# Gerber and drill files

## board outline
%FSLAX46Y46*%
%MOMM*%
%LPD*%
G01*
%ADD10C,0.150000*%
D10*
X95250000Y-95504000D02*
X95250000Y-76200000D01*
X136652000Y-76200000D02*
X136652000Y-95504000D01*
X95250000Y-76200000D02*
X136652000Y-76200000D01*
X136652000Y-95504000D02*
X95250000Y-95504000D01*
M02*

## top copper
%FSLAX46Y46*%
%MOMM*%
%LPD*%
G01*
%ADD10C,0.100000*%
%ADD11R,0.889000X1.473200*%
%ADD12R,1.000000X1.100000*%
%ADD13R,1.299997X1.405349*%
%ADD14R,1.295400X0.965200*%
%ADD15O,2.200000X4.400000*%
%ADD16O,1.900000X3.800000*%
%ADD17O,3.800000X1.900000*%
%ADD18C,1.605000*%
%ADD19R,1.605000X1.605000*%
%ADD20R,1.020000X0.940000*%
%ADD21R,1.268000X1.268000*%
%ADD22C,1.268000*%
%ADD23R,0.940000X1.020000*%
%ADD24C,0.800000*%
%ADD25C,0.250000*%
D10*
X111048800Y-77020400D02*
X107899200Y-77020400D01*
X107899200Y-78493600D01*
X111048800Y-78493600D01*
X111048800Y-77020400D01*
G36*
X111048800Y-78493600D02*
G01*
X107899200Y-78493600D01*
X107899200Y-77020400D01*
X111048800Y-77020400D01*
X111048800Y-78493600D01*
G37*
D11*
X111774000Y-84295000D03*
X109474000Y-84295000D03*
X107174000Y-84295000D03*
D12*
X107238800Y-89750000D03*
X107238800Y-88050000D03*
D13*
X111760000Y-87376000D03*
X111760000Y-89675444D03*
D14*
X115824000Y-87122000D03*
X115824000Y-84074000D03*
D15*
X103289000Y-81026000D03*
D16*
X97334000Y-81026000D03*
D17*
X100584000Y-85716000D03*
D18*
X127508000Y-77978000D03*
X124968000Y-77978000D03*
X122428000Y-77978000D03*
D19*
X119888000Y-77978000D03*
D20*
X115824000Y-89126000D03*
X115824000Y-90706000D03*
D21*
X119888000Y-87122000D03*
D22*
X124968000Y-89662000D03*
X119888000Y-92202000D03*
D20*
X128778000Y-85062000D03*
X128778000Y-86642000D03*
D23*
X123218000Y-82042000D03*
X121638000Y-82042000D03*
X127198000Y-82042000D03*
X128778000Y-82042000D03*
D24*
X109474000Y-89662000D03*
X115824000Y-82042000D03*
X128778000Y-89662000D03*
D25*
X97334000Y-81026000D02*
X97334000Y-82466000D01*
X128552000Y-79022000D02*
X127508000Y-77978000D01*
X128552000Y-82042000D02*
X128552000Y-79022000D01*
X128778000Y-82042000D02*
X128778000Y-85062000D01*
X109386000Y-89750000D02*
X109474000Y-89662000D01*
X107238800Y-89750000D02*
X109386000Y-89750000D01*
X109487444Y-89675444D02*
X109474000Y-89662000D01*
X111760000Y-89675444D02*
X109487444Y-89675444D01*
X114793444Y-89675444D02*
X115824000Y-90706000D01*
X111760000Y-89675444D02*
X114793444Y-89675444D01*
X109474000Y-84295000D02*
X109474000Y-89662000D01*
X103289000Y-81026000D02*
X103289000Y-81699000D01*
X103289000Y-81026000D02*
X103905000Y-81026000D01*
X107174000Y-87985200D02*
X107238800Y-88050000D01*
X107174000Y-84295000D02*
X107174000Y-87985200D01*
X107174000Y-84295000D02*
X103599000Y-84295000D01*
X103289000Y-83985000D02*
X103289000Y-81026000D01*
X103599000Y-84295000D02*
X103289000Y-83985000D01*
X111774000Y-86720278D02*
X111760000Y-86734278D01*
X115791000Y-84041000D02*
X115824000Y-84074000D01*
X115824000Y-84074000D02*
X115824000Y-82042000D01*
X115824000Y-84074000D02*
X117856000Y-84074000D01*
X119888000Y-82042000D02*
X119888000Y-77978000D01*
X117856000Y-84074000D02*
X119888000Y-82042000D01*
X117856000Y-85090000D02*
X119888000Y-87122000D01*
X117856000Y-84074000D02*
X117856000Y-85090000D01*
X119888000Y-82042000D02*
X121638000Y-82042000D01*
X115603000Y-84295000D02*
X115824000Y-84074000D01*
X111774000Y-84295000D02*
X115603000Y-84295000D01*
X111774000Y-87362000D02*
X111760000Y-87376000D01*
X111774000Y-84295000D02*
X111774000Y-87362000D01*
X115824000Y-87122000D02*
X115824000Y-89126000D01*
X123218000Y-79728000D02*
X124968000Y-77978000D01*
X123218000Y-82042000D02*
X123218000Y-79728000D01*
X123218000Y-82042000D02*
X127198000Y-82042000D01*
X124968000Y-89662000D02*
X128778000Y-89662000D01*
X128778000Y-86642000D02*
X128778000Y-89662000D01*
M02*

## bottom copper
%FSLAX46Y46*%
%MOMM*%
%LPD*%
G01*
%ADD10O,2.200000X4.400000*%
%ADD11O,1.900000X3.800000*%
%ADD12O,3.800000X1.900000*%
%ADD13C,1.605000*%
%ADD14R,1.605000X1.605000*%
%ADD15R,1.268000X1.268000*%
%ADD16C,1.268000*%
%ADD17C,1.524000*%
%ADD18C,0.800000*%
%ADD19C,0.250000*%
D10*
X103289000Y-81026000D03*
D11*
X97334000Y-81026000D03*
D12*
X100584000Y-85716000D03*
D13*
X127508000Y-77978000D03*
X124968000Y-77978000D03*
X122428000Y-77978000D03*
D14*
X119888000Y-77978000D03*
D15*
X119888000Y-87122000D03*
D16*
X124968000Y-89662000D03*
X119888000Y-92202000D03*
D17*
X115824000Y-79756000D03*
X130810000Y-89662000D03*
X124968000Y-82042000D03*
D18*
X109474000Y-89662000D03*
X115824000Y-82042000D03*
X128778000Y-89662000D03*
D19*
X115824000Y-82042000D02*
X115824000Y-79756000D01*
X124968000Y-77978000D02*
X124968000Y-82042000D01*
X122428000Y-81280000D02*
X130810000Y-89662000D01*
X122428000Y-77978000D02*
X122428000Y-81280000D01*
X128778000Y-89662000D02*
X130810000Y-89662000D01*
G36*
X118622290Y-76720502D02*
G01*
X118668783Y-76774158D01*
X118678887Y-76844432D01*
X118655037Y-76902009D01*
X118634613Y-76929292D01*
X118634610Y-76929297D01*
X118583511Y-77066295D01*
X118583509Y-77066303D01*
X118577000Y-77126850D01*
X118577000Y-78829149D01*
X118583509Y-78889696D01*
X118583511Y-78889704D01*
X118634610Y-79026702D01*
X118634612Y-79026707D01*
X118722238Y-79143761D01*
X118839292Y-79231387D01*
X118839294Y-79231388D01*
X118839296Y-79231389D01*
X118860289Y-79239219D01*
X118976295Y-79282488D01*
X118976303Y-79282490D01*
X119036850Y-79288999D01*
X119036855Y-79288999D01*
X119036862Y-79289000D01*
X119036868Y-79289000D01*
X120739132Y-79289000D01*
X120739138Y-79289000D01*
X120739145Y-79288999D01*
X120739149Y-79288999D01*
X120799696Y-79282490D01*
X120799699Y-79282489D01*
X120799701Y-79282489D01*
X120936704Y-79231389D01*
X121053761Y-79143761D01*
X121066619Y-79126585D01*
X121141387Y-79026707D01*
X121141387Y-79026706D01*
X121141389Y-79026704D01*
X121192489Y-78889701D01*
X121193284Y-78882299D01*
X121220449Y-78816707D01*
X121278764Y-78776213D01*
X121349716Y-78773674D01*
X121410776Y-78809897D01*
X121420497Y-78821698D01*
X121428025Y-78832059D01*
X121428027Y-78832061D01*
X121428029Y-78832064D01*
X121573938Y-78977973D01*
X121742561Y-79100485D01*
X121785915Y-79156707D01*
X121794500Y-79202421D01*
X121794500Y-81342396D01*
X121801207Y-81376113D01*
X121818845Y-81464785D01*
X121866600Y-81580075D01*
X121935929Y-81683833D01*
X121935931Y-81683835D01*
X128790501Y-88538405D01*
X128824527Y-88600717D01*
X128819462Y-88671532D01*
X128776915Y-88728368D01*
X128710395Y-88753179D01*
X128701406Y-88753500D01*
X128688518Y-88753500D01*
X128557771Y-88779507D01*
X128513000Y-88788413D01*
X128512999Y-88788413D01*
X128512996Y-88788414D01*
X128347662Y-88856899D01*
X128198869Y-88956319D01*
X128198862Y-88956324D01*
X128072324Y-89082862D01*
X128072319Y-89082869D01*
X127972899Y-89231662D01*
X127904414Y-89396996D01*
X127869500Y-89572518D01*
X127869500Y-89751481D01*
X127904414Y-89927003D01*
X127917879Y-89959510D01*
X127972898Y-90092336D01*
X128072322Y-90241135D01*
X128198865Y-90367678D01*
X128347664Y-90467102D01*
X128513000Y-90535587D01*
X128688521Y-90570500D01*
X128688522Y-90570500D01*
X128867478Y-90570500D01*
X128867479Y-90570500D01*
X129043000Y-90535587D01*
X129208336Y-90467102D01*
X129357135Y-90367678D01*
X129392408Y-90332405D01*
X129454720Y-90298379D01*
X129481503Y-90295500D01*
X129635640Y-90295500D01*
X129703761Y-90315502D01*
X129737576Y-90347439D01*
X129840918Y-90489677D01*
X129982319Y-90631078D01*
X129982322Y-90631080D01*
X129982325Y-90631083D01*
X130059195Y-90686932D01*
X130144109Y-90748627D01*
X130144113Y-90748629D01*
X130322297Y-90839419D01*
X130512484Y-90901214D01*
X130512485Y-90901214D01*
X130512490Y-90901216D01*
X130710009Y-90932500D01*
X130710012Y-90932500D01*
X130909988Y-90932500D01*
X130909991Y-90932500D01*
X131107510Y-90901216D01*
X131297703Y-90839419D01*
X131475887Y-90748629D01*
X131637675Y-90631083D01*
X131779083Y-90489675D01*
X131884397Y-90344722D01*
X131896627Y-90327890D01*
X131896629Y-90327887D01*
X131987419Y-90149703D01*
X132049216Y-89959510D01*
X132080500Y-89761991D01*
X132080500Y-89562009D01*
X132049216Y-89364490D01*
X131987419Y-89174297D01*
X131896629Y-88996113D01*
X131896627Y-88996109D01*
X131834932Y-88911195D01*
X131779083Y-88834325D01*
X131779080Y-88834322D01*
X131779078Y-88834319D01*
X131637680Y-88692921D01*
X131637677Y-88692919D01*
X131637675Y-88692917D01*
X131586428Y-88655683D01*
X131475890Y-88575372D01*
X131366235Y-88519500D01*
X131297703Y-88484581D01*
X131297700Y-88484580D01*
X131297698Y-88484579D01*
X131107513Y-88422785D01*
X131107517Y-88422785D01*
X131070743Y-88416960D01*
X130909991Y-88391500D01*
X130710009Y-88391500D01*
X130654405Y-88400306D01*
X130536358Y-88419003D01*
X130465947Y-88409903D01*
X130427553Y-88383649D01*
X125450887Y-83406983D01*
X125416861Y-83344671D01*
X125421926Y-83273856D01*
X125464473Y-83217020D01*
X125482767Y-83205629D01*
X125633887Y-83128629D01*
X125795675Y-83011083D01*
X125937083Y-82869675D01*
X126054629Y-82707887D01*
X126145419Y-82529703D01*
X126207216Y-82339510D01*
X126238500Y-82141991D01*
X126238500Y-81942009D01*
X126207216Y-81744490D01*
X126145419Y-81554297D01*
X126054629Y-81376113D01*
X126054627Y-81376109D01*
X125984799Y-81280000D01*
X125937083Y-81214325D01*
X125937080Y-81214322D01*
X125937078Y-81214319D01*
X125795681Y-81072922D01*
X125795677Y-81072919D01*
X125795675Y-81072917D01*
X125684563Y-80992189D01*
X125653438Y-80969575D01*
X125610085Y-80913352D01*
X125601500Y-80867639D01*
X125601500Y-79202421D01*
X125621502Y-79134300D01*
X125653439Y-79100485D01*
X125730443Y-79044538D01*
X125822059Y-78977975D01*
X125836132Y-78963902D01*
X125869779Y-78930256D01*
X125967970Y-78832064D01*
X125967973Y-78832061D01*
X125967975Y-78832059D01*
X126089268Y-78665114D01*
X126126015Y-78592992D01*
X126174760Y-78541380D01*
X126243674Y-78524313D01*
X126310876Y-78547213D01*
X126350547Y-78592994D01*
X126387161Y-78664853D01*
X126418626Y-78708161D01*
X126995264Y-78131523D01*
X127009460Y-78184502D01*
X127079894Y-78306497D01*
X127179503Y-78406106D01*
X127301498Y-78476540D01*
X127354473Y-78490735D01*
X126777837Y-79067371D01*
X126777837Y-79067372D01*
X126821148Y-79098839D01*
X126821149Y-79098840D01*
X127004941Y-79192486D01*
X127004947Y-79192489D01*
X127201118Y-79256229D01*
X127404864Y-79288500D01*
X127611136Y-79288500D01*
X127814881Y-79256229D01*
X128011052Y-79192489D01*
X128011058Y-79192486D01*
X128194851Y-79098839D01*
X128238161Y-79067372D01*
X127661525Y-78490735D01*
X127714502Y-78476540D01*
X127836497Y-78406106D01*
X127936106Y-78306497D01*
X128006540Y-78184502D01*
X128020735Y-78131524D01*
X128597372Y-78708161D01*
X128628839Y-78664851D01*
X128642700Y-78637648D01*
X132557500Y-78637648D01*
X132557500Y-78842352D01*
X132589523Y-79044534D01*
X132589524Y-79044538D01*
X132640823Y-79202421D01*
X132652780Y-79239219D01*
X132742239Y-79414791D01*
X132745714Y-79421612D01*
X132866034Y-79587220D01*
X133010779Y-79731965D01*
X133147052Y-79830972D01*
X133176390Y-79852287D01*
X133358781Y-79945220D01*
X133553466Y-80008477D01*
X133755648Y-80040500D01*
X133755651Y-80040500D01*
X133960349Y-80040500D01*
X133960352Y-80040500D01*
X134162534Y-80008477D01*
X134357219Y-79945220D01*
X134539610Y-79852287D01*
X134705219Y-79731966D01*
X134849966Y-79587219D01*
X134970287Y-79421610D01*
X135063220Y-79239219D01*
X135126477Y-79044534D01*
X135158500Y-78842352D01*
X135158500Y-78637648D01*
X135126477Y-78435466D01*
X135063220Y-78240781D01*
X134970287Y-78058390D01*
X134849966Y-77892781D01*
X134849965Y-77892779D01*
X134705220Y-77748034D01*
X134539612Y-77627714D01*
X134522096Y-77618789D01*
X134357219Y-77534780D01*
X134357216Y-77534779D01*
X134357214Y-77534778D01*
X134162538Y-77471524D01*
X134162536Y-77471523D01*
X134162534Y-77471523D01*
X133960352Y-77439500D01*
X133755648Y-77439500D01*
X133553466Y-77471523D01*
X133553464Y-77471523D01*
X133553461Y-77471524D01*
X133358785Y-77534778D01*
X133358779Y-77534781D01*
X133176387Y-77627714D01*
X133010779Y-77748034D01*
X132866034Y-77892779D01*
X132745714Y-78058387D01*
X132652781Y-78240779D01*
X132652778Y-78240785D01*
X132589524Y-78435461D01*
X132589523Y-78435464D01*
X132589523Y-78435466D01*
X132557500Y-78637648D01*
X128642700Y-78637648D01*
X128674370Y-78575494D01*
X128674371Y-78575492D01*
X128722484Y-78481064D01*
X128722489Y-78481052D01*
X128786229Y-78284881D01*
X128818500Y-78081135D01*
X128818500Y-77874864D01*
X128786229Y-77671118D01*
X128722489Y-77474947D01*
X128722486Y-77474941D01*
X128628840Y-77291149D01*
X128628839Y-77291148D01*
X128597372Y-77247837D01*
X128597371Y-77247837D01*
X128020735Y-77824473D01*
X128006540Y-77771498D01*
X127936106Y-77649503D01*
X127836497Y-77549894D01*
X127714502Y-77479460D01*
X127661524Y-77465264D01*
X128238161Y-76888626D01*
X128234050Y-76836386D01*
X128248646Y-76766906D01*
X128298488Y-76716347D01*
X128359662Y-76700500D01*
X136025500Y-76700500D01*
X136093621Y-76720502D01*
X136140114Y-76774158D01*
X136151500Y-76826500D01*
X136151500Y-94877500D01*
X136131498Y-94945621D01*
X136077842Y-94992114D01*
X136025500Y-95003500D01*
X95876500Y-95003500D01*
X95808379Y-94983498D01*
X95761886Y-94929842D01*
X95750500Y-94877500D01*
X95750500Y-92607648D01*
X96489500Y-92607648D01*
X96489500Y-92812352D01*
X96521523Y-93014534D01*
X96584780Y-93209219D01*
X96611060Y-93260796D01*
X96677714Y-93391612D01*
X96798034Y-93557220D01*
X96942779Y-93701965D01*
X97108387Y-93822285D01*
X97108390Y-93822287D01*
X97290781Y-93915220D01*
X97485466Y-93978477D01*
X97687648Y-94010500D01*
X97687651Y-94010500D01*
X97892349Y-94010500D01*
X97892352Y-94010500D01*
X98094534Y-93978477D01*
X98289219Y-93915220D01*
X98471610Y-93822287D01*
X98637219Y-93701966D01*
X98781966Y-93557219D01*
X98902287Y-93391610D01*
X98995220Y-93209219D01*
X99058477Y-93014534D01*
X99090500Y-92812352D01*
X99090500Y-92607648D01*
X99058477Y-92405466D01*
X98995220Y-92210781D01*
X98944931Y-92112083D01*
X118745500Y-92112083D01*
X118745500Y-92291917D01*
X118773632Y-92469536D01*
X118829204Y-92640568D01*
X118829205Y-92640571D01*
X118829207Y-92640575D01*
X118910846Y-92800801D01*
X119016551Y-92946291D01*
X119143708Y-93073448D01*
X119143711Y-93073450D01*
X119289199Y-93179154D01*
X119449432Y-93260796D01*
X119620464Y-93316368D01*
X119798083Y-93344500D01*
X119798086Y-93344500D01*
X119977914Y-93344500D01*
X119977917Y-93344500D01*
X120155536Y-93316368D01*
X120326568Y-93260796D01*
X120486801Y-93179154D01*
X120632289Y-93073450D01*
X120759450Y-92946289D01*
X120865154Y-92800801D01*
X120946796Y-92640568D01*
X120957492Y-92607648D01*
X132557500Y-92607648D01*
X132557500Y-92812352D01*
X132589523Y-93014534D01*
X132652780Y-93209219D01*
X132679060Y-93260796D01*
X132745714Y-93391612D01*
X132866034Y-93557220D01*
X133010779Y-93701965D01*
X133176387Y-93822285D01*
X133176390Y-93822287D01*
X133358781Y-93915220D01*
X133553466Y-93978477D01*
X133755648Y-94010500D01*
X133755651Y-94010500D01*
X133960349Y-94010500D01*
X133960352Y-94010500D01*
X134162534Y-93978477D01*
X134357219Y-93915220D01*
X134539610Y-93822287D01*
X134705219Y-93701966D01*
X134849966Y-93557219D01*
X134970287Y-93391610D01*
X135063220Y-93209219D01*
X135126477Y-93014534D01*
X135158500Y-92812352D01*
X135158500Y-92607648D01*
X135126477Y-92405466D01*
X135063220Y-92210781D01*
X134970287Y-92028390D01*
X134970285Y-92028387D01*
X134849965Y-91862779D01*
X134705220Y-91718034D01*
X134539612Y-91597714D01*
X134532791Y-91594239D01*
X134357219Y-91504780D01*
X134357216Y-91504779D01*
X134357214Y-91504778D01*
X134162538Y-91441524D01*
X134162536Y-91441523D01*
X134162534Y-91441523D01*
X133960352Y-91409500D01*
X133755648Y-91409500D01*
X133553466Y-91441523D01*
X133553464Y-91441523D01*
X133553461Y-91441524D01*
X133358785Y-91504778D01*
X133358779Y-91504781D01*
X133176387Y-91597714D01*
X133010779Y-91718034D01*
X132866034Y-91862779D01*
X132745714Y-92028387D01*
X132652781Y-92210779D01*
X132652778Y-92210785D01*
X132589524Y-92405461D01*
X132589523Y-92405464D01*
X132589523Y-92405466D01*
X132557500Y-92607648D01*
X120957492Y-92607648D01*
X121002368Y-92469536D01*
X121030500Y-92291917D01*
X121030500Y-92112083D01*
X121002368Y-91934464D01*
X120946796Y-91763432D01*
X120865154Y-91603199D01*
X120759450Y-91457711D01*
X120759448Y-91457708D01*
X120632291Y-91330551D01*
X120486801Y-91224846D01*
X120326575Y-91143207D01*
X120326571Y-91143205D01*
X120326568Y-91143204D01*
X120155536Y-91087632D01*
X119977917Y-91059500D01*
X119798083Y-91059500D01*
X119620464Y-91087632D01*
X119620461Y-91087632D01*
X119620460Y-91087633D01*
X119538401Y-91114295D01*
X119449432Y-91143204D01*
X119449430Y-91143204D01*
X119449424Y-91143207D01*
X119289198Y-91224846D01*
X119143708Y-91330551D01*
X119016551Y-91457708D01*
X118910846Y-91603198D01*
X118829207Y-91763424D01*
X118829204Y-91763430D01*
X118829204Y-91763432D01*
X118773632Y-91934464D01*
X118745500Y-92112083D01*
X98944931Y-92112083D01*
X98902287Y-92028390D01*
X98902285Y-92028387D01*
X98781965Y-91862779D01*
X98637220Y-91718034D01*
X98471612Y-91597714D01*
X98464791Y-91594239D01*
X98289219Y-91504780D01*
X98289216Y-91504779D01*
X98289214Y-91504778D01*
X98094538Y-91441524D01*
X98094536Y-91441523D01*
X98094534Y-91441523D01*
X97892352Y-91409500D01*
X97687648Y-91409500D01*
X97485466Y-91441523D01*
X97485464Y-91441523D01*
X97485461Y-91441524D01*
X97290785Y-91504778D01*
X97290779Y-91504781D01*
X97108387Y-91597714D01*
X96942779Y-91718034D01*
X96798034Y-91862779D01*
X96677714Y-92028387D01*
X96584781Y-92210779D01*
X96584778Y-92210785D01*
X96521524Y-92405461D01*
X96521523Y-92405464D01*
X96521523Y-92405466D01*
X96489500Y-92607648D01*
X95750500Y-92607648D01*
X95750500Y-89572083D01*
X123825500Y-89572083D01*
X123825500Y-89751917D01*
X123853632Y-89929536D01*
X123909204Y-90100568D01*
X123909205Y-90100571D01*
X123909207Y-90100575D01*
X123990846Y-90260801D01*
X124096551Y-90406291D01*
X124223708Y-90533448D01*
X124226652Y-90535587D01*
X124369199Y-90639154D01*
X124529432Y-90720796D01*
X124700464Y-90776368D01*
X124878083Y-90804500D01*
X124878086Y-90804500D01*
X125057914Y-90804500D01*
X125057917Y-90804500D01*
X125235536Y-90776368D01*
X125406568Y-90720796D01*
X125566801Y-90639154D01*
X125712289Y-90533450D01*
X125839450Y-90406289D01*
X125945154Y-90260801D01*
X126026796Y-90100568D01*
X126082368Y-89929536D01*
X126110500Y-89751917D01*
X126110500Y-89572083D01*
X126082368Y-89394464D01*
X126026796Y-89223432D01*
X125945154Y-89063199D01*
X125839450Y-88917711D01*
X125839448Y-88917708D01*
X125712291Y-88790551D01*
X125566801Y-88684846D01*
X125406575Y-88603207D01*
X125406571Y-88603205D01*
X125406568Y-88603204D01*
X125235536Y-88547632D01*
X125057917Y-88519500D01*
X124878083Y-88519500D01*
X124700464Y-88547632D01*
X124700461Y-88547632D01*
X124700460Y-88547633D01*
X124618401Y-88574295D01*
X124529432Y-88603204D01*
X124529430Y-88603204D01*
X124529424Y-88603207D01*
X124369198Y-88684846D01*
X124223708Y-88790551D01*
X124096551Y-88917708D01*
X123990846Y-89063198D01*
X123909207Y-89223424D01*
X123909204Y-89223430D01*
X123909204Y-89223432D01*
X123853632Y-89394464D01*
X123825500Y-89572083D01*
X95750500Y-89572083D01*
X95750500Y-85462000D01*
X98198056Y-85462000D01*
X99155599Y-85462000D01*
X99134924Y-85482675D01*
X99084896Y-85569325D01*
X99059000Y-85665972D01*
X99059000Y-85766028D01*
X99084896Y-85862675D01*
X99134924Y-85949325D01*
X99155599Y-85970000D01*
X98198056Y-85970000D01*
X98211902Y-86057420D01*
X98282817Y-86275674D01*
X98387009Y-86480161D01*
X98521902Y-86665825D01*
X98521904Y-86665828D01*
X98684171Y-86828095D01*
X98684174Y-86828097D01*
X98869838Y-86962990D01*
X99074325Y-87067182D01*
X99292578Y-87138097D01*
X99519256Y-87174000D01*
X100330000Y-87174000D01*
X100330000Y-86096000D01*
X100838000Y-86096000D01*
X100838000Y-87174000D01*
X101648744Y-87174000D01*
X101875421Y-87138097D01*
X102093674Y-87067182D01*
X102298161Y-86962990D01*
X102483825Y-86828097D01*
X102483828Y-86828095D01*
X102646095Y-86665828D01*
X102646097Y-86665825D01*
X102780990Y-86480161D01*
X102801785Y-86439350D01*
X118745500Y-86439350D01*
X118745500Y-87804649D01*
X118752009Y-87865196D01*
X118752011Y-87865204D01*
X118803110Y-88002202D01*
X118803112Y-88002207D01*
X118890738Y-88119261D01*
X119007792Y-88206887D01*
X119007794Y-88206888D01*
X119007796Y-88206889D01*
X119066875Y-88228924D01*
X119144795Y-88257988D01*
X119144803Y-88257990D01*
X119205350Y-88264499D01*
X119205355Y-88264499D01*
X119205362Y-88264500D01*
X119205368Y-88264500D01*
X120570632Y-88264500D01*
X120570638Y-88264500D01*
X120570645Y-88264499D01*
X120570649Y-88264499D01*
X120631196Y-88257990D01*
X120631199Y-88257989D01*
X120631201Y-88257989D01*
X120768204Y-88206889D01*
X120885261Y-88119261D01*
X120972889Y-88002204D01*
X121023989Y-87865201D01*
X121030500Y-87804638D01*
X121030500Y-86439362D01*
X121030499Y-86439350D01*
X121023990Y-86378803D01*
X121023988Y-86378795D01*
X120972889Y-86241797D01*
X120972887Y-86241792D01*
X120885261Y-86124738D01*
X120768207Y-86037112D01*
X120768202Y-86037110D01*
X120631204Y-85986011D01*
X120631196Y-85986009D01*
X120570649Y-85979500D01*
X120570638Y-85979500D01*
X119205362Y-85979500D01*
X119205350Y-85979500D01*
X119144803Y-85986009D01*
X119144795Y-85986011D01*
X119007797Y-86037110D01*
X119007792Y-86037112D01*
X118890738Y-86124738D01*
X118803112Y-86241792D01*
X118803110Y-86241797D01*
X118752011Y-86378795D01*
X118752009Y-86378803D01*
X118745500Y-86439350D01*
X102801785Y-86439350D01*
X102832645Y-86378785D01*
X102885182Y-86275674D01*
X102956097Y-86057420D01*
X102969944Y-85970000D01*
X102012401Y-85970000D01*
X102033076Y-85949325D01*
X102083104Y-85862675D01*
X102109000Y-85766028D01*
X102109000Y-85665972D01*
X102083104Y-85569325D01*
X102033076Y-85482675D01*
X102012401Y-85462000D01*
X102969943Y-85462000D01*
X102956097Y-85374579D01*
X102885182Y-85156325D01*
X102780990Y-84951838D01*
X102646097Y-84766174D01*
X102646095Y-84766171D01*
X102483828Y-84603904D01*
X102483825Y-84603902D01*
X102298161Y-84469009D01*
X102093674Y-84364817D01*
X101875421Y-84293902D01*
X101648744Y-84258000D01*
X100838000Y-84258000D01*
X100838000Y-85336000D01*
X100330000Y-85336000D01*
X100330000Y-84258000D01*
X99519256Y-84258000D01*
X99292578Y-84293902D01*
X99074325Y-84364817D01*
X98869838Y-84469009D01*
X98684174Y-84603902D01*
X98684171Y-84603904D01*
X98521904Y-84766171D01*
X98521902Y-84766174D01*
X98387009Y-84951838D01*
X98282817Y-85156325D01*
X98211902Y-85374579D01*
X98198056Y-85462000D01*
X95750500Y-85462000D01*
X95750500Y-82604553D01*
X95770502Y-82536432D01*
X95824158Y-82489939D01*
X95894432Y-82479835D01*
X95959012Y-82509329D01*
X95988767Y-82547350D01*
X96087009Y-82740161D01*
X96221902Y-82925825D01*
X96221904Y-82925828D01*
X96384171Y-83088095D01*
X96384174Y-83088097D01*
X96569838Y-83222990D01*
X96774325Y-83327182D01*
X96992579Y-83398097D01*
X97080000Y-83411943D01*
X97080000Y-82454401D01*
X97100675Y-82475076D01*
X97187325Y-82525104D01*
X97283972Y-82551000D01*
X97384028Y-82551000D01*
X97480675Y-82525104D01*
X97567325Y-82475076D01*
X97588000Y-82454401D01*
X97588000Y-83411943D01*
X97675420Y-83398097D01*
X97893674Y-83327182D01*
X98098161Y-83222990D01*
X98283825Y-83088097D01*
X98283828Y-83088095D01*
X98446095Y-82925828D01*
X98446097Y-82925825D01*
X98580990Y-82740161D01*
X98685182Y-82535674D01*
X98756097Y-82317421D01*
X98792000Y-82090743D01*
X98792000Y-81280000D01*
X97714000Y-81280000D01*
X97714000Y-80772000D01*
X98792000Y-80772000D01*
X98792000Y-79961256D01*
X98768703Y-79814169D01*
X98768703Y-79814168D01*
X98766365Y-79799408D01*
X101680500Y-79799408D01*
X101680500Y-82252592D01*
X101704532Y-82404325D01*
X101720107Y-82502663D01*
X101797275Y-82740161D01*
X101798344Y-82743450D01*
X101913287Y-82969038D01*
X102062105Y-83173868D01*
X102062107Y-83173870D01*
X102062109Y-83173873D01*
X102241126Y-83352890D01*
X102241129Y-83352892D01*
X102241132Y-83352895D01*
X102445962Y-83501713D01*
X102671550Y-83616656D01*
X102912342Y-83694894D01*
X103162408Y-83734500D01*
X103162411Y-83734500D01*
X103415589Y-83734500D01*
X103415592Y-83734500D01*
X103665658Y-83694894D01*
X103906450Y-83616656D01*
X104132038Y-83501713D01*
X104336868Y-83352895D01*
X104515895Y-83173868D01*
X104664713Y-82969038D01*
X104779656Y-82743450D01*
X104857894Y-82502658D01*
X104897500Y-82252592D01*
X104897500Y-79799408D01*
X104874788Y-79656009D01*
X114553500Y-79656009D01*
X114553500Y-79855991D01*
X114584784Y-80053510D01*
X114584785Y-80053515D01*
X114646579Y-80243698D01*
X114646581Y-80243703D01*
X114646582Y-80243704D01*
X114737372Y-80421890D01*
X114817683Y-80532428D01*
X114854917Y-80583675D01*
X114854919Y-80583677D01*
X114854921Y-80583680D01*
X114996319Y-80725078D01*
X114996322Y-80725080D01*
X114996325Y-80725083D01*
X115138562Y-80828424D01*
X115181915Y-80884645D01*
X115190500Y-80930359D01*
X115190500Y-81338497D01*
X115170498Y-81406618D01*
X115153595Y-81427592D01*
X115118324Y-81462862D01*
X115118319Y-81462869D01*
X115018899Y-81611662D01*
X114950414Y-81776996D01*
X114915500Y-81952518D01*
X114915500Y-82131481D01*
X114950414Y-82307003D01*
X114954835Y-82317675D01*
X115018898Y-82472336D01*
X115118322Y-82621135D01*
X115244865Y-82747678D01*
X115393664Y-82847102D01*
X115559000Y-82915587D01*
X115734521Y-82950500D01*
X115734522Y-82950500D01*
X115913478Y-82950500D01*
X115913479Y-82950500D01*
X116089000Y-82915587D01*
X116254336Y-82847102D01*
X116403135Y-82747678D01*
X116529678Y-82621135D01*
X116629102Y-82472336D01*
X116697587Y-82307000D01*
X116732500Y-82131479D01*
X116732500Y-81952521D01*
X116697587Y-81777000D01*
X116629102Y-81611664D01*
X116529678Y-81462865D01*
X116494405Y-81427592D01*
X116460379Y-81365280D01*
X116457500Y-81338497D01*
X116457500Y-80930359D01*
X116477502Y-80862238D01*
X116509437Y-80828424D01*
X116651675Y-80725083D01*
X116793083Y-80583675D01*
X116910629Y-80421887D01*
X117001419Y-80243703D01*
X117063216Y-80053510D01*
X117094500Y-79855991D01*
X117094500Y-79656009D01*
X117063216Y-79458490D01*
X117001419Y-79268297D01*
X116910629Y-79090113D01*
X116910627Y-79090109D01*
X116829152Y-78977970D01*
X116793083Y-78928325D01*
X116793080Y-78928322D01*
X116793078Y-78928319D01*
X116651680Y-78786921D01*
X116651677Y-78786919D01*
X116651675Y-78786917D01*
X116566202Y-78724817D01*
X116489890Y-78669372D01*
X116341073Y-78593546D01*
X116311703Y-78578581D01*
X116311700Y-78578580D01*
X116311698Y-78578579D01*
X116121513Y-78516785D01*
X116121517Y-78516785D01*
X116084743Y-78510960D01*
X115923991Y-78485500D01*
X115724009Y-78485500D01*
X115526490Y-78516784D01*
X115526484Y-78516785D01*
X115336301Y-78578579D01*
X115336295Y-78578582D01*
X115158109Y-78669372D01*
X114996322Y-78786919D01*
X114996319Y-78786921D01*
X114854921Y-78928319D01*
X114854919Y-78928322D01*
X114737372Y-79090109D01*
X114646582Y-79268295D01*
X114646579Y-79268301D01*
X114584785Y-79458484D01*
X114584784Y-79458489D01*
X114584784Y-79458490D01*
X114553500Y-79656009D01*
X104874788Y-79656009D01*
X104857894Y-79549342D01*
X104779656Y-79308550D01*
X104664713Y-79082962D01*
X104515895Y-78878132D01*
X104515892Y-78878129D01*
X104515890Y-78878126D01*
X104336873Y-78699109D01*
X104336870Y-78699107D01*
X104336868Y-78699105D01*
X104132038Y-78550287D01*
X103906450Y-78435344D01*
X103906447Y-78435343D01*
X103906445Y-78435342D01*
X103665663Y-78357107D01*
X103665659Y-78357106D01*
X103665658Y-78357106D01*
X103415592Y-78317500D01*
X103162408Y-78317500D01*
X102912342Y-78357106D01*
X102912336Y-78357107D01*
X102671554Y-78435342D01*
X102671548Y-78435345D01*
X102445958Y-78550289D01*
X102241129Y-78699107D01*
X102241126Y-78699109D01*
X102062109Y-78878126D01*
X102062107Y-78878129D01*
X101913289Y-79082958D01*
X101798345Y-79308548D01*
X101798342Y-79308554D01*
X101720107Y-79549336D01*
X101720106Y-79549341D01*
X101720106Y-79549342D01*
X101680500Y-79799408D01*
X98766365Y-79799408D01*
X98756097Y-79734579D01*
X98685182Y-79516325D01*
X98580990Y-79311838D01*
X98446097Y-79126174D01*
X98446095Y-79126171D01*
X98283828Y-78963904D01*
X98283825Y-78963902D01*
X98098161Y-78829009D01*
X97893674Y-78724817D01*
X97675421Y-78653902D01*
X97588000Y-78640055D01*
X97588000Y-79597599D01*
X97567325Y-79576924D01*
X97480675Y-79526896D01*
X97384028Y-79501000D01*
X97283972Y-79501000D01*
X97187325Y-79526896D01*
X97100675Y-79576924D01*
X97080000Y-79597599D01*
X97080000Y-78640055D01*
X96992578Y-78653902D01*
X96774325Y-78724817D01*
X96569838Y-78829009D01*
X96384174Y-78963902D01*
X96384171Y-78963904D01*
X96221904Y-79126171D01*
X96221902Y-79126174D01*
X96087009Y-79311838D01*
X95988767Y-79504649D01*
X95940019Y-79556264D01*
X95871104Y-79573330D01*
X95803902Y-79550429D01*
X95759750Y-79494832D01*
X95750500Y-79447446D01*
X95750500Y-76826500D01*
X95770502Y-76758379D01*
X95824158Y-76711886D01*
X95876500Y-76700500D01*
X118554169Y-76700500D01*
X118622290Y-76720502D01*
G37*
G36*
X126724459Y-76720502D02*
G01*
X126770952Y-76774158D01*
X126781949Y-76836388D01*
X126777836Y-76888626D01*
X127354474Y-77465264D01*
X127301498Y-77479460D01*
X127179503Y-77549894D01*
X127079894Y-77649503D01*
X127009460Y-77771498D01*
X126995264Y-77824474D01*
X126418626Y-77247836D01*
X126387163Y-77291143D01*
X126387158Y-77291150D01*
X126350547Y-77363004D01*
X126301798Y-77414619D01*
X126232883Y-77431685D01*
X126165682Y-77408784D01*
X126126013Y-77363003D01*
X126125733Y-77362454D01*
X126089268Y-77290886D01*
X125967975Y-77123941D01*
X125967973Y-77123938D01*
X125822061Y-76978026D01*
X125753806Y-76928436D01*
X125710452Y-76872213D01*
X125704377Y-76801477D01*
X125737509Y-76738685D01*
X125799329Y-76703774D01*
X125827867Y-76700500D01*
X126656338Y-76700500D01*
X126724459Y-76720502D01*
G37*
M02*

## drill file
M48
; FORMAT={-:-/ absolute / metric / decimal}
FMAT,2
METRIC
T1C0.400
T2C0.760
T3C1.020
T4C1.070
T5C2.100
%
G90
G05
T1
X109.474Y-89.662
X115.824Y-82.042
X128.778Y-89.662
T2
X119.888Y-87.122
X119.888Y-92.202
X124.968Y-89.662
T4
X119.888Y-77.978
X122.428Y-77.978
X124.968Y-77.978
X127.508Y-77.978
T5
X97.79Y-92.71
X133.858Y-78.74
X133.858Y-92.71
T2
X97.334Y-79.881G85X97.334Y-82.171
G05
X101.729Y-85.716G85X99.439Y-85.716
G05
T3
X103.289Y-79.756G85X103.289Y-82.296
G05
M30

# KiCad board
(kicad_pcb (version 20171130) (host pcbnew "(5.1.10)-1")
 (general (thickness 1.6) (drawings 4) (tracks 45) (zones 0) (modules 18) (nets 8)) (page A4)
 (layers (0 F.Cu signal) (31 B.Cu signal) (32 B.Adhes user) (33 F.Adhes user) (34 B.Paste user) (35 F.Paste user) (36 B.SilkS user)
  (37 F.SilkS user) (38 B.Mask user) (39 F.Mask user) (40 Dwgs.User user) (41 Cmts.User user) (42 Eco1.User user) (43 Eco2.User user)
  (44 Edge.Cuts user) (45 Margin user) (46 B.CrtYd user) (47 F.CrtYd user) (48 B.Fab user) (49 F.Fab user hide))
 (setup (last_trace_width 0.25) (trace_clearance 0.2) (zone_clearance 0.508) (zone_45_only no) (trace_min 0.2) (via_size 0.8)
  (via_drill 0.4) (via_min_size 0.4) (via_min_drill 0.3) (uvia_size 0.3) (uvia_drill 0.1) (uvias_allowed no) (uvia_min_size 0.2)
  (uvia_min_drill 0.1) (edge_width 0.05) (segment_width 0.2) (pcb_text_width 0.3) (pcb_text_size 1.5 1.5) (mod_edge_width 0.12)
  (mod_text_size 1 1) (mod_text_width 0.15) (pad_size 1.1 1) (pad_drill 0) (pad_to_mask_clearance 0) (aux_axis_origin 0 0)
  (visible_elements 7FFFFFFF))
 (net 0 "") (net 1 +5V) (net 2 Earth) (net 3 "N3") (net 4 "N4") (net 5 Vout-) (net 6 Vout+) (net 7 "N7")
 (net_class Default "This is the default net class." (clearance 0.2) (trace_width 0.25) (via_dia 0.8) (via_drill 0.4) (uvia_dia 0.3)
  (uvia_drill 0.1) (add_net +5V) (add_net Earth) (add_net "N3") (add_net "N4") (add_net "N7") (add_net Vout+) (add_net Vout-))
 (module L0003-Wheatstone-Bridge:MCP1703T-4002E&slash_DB (layer F.Cu) (at 109.474 81.026)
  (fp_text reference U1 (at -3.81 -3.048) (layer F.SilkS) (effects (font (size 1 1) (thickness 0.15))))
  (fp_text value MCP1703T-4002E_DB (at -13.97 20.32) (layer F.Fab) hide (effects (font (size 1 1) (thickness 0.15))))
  (fp_poly (pts (xy 1.5748 -4.0056) (xy -1.5748 -4.0056) (xy -1.5748 -2.5324) (xy 1.5748 -2.5324)) (layer F.Cu) (width 0.1))
  (pad 3 smd rect (at 2.3 3.269) (size 0.889 1.4732) (layers F.Cu F.Paste F.Mask) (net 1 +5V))
  (pad 2 smd rect (at 0 3.269) (size 0.889 1.4732) (layers F.Cu F.Paste F.Mask) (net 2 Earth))
  (pad 1 smd rect (at -2.3 3.269) (size 0.889 1.4732) (layers F.Cu F.Paste F.Mask) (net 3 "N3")))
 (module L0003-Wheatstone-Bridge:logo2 (layer F.Cu) (at 105.156 92.71)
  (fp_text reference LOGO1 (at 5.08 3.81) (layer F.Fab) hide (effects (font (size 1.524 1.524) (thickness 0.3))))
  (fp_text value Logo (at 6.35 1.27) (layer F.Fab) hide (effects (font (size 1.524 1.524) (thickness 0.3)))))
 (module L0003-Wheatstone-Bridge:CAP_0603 (layer F.Cu) (at 107.2388 88.9 90)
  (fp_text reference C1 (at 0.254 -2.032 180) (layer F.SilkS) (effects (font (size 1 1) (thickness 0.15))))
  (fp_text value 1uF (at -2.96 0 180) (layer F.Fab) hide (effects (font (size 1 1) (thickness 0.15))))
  (pad 1 smd rect (at -0.85 0 90) (size 1.1 1) (layers F.Cu F.Paste F.Mask) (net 2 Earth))
  (pad 2 smd rect (at 0.85 0 90) (size 1.1 1) (layers F.Cu F.Paste F.Mask) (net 3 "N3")))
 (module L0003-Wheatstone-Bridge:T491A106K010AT (layer F.Cu) (at 111.76 88.525722 270)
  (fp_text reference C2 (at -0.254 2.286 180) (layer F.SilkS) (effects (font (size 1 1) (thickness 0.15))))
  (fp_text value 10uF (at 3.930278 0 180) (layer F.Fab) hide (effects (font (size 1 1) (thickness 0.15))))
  (pad 1 smd rect (at -1.149722 0) (size 1.299997 1.405349) (layers F.Cu F.Paste F.Mask) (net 1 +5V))
  (pad 2 smd rect (at 1.149722 0) (size 1.299997 1.405349) (layers F.Cu F.Paste F.Mask) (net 2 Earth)))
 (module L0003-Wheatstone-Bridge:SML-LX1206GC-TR (layer F.Cu) (at 115.824 85.598 90)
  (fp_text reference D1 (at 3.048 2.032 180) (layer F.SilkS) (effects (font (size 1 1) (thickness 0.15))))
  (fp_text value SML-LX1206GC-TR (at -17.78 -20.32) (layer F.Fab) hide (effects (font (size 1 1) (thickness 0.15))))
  (pad 1 smd rect (at -1.524 0 90) (size 0.9652 1.2954) (layers F.Cu F.Paste F.Mask) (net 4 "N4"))
  (pad 2 smd rect (at 1.524 0 90) (size 0.9652 1.2954) (layers F.Cu F.Paste F.Mask) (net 1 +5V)))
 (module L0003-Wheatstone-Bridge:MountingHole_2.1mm (layer F.Cu) (at 133.858 92.71)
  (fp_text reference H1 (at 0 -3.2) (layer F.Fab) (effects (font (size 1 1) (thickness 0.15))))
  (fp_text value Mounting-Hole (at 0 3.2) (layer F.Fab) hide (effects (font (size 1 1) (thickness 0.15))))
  (pad "" np_thru_hole circle (at 0 0) (size 2.1 2.1) (drill 2.1) (layers *.Cu *.Mask)))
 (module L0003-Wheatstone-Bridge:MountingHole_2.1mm (layer F.Cu) (at 133.858 78.74)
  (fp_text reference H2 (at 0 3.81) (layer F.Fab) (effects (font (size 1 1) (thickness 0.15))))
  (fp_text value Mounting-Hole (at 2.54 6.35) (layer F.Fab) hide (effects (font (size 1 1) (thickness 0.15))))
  (pad "" np_thru_hole circle (at 0 0) (size 2.1 2.1) (drill 2.1) (layers *.Cu *.Mask)))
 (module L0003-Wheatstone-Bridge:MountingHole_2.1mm (layer F.Cu) (at 97.79 92.71)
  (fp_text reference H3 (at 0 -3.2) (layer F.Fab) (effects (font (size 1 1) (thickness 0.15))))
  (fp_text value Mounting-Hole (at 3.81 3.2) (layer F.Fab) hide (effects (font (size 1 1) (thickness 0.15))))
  (pad "" np_thru_hole circle (at 0 0) (size 2.1 2.1) (drill 2.1) (layers *.Cu *.Mask)))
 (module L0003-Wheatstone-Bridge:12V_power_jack (layer F.Cu) (at 100.584 81.026 270)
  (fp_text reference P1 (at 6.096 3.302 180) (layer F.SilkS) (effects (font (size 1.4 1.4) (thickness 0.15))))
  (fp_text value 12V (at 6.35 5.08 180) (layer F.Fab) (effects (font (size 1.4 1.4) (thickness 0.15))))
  (pad 1 thru_hole oval (at 0 -2.705 270) (size 4.4 2.2) (drill oval 3.56 1.02) (layers *.Cu *.Mask) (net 3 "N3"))
  (pad 2 thru_hole oval (at 0 3.25 270) (size 3.8 1.9) (drill oval 3.05 0.76) (layers *.Cu *.Mask) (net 2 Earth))
  (pad 3 thru_hole oval (at 4.69 0 270) (size 1.9 3.8) (drill oval 0.76 3.05) (layers *.Cu *.Mask) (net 2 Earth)))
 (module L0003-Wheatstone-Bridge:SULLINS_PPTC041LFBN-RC (layer F.Cu) (at 123.698 77.978)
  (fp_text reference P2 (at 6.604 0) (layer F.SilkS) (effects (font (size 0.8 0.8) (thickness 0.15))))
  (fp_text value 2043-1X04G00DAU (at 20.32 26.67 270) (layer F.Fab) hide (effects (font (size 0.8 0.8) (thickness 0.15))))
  (pad 4 thru_hole circle (at 3.81 0) (size 1.605 1.605) (drill 1.07) (layers *.Cu *.Mask) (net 2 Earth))
  (pad 3 thru_hole circle (at 1.27 0) (size 1.605 1.605) (drill 1.07) (layers *.Cu *.Mask) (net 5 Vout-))
  (pad 2 thru_hole circle (at -1.27 0) (size 1.605 1.605) (drill 1.07) (layers *.Cu *.Mask) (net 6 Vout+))
  (pad 1 thru_hole rect (at -3.81 0) (size 1.605 1.605) (drill 1.07) (layers *.Cu *.Mask) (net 1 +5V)))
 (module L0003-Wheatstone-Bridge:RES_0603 (layer F.Cu) (at 115.824 89.916 270)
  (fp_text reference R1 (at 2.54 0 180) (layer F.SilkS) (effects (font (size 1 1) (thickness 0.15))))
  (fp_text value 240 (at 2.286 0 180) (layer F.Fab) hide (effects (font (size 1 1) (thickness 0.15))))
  (pad 1 smd rect (at -0.79 0 270) (size 0.94 1.02) (layers F.Cu F.Paste F.Mask) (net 4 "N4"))
  (pad 2 smd rect (at 0.79 0 270) (size 0.94 1.02) (layers F.Cu F.Paste F.Mask) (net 2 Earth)))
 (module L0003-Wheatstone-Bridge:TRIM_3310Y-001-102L (layer F.Cu) (at 122.428 89.662 270)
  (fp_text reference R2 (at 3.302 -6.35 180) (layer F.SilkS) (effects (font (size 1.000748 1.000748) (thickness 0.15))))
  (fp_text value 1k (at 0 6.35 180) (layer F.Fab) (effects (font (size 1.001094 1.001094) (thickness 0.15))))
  (pad 1 thru_hole rect (at -2.54 2.54 270) (size 1.268 1.268) (drill 0.76) (layers *.Cu *.Mask) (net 1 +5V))
  (pad 2 thru_hole circle (at 0 -2.54 270) (size 1.268 1.268) (drill 0.76) (layers *.Cu *.Mask) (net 6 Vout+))
  (pad 3 thru_hole circle (at 2.54 2.54 270) (size 1.268 1.268) (drill 0.76) (layers *.Cu *.Mask) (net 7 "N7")))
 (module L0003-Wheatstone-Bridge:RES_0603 (layer F.Cu) (at 128.778 85.852 90)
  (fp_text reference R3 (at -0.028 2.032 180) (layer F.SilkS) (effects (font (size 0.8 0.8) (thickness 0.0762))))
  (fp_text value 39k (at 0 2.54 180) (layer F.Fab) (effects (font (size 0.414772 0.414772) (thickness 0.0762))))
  (pad 2 smd rect (at 0.79 0 90) (size 0.94 1.02) (layers F.Cu F.Paste F.Mask) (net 2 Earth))
  (pad 1 smd rect (at -0.79 0 90) (size 0.94 1.02) (layers F.Cu F.Paste F.Mask) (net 6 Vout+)))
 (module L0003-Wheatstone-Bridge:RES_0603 (layer F.Cu) (at 122.428 82.042)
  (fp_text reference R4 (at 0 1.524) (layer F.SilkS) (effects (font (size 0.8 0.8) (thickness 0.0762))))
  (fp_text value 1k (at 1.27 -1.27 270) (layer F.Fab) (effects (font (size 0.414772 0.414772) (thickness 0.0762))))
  (pad 2 smd rect (at 0.79 0) (size 0.94 1.02) (layers F.Cu F.Paste F.Mask) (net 5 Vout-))
  (pad 1 smd rect (at -0.79 0) (size 0.94 1.02) (layers F.Cu F.Paste F.Mask) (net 1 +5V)))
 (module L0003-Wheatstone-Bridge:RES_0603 (layer F.Cu) (at 127.988 82.042)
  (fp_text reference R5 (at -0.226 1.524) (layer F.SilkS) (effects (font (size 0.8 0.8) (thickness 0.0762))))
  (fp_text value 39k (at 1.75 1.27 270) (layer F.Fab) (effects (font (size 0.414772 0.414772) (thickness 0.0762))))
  (pad 1 smd rect (at -0.79 0) (size 0.94 1.02) (layers F.Cu F.Paste F.Mask) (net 5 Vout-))
  (pad 2 smd rect (at 0.79 0) (size 0.94 1.02) (layers F.Cu F.Paste F.Mask) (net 2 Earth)))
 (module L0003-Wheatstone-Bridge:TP (layer B.Cu) (at 115.824 79.756)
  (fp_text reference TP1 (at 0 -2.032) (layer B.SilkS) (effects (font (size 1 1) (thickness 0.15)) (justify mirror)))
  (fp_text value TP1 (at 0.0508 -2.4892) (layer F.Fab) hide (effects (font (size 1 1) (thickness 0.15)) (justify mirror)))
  (pad 1 smd circle (at 0 0) (size 1.524 1.524) (layers B.Cu B.Paste B.Mask) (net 1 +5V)))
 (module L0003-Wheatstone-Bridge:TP (layer B.Cu) (at 130.81 89.662)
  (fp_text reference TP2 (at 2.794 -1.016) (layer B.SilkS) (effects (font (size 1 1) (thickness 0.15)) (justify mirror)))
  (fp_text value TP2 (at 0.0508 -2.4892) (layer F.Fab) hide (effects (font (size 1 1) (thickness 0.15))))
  (pad 1 smd circle (at 0 0) (size 1.524 1.524) (layers B.Cu B.Paste B.Mask) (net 6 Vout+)))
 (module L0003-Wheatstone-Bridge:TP (layer B.Cu) (at 124.968 82.042)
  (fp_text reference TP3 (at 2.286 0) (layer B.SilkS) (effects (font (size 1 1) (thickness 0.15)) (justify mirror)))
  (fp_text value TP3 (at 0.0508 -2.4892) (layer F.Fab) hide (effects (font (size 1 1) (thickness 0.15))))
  (pad 1 smd circle (at 0 0) (size 1.524 1.524) (layers B.Cu B.Paste B.Mask) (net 5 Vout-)))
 (gr_line (start 95.25 95.504) (end 95.25 76.2) (layer Edge.Cuts) (width 0.15))
 (gr_line (start 136.652 76.2) (end 136.652 95.504) (layer Edge.Cuts) (width 0.15))
 (gr_line (start 95.25 76.2) (end 136.652 76.2) (layer Edge.Cuts) (width 0.15))
 (gr_line (start 136.652 95.504) (end 95.25 95.504) (layer Edge.Cuts) (width 0.15))
 (via (at 109.474 89.662) (size 0.8) (drill 0.4) (layers F.Cu B.Cu) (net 2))
 (segment (start 97.334 81.026) (end 97.334 82.466) (width 0.25) (layer F.Cu) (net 2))
 (segment (start 128.552 79.022) (end 127.508 77.978) (width 0.25) (layer F.Cu) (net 2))
 (segment (start 128.552 82.042) (end 128.552 79.022) (width 0.25) (layer F.Cu) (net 2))
 (segment (start 128.778 82.042) (end 128.778 85.062) (width 0.25) (layer F.Cu) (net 2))
 (segment (start 109.386 89.75) (end 109.474 89.662) (width 0.25) (layer F.Cu) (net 2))
 (segment (start 107.2388 89.75) (end 109.386 89.75) (width 0.25) (layer F.Cu) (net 2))
 (segment (start 109.487444 89.675444) (end 109.474 89.662) (width 0.25) (layer F.Cu) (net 2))
 (segment (start 111.76 89.675444) (end 109.487444 89.675444) (width 0.25) (layer F.Cu) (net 2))
 (segment (start 114.793444 89.675444) (end 115.824 90.706) (width 0.25) (layer F.Cu) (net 2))
 (segment (start 111.76 89.675444) (end 114.793444 89.675444) (width 0.25) (layer F.Cu) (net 2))
 (segment (start 109.474 84.295) (end 109.474 89.662) (width 0.25) (layer F.Cu) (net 2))
 (segment (start 103.289 81.026) (end 103.289 81.699) (width 0.25) (layer F.Cu) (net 3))
 (segment (start 103.289 81.026) (end 103.905 81.026) (width 0.25) (layer F.Cu) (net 3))
 (segment (start 107.174 87.9852) (end 107.2388 88.05) (width 0.25) (layer F.Cu) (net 3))
 (segment (start 107.174 84.295) (end 107.174 87.9852) (width 0.25) (layer F.Cu) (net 3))
 (segment (start 107.174 84.295) (end 103.599 84.295) (width 0.25) (layer F.Cu) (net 3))
 (segment (start 103.289 83.985) (end 103.289 81.026) (width 0.25) (layer F.Cu) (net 3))
 (segment (start 103.599 84.295) (end 103.289 83.985) (width 0.25) (layer F.Cu) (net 3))
 (via (at 115.824 82.042) (size 0.8) (drill 0.4) (layers F.Cu B.Cu) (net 1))
 (segment (start 111.774 86.720278) (end 111.76 86.734278) (width 0.25) (layer F.Cu) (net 1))
 (segment (start 115.791 84.041) (end 115.824 84.074) (width 0.25) (layer F.Cu) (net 1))
 (segment (start 115.824 84.074) (end 115.824 82.042) (width 0.25) (layer F.Cu) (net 1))
 (segment (start 115.824 82.042) (end 115.824 79.756) (width 0.25) (layer B.Cu) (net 1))
 (segment (start 115.824 84.074) (end 117.856 84.074) (width 0.25) (layer F.Cu) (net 1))
 (segment (start 119.888 82.042) (end 119.888 77.978) (width 0.25) (layer F.Cu) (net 1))
 (segment (start 117.856 84.074) (end 119.888 82.042) (width 0.25) (layer F.Cu) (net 1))
 (segment (start 117.856 85.09) (end 119.888 87.122) (width 0.25) (layer F.Cu) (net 1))
 (segment (start 117.856 84.074) (end 117.856 85.09) (width 0.25) (layer F.Cu) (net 1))
 (segment (start 119.888 82.042) (end 121.638 82.042) (width 0.25) (layer F.Cu) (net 1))
 (segment (start 115.603 84.295) (end 115.824 84.074) (width 0.25) (layer F.Cu) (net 1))
 (segment (start 111.774 84.295) (end 115.603 84.295) (width 0.25) (layer F.Cu) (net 1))
 (segment (start 111.774 87.362) (end 111.76 87.376) (width 0.25) (layer F.Cu) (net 1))
 (segment (start 111.774 84.295) (end 111.774 87.362) (width 0.25) (layer F.Cu) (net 1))
 (segment (start 115.824 87.122) (end 115.824 89.126) (width 0.25) (layer F.Cu) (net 4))
 (segment (start 123.218 79.728) (end 124.968 77.978) (width 0.25) (layer F.Cu) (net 5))
 (segment (start 123.218 82.042) (end 123.218 79.728) (width 0.25) (layer F.Cu) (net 5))
 (segment (start 124.968 77.978) (end 124.968 82.042) (width 0.25) (layer B.Cu) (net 5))
 (segment (start 123.218 82.042) (end 127.198 82.042) (width 0.25) (layer F.Cu) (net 5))
 (via (at 128.778 89.662) (size 0.8) (drill 0.4) (layers F.Cu B.Cu) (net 6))
 (segment (start 122.428 81.28) (end 130.81 89.662) (width 0.25) (layer B.Cu) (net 6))
 (segment (start 122.428 77.978) (end 122.428 81.28) (width 0.25) (layer B.Cu) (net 6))
 (segment (start 124.968 89.662) (end 128.778 89.662) (width 0.25) (layer F.Cu) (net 6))
 (segment (start 128.778 86.642) (end 128.778 89.662) (width 0.25) (layer F.Cu) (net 6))
 (segment (start 128.778 89.662) (end 130.81 89.662) (width 0.25) (layer B.Cu) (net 6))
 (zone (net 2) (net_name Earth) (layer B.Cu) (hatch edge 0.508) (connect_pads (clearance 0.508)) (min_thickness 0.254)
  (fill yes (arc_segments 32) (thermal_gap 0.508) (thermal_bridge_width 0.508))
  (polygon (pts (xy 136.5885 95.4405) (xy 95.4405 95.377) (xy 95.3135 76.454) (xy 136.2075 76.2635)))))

